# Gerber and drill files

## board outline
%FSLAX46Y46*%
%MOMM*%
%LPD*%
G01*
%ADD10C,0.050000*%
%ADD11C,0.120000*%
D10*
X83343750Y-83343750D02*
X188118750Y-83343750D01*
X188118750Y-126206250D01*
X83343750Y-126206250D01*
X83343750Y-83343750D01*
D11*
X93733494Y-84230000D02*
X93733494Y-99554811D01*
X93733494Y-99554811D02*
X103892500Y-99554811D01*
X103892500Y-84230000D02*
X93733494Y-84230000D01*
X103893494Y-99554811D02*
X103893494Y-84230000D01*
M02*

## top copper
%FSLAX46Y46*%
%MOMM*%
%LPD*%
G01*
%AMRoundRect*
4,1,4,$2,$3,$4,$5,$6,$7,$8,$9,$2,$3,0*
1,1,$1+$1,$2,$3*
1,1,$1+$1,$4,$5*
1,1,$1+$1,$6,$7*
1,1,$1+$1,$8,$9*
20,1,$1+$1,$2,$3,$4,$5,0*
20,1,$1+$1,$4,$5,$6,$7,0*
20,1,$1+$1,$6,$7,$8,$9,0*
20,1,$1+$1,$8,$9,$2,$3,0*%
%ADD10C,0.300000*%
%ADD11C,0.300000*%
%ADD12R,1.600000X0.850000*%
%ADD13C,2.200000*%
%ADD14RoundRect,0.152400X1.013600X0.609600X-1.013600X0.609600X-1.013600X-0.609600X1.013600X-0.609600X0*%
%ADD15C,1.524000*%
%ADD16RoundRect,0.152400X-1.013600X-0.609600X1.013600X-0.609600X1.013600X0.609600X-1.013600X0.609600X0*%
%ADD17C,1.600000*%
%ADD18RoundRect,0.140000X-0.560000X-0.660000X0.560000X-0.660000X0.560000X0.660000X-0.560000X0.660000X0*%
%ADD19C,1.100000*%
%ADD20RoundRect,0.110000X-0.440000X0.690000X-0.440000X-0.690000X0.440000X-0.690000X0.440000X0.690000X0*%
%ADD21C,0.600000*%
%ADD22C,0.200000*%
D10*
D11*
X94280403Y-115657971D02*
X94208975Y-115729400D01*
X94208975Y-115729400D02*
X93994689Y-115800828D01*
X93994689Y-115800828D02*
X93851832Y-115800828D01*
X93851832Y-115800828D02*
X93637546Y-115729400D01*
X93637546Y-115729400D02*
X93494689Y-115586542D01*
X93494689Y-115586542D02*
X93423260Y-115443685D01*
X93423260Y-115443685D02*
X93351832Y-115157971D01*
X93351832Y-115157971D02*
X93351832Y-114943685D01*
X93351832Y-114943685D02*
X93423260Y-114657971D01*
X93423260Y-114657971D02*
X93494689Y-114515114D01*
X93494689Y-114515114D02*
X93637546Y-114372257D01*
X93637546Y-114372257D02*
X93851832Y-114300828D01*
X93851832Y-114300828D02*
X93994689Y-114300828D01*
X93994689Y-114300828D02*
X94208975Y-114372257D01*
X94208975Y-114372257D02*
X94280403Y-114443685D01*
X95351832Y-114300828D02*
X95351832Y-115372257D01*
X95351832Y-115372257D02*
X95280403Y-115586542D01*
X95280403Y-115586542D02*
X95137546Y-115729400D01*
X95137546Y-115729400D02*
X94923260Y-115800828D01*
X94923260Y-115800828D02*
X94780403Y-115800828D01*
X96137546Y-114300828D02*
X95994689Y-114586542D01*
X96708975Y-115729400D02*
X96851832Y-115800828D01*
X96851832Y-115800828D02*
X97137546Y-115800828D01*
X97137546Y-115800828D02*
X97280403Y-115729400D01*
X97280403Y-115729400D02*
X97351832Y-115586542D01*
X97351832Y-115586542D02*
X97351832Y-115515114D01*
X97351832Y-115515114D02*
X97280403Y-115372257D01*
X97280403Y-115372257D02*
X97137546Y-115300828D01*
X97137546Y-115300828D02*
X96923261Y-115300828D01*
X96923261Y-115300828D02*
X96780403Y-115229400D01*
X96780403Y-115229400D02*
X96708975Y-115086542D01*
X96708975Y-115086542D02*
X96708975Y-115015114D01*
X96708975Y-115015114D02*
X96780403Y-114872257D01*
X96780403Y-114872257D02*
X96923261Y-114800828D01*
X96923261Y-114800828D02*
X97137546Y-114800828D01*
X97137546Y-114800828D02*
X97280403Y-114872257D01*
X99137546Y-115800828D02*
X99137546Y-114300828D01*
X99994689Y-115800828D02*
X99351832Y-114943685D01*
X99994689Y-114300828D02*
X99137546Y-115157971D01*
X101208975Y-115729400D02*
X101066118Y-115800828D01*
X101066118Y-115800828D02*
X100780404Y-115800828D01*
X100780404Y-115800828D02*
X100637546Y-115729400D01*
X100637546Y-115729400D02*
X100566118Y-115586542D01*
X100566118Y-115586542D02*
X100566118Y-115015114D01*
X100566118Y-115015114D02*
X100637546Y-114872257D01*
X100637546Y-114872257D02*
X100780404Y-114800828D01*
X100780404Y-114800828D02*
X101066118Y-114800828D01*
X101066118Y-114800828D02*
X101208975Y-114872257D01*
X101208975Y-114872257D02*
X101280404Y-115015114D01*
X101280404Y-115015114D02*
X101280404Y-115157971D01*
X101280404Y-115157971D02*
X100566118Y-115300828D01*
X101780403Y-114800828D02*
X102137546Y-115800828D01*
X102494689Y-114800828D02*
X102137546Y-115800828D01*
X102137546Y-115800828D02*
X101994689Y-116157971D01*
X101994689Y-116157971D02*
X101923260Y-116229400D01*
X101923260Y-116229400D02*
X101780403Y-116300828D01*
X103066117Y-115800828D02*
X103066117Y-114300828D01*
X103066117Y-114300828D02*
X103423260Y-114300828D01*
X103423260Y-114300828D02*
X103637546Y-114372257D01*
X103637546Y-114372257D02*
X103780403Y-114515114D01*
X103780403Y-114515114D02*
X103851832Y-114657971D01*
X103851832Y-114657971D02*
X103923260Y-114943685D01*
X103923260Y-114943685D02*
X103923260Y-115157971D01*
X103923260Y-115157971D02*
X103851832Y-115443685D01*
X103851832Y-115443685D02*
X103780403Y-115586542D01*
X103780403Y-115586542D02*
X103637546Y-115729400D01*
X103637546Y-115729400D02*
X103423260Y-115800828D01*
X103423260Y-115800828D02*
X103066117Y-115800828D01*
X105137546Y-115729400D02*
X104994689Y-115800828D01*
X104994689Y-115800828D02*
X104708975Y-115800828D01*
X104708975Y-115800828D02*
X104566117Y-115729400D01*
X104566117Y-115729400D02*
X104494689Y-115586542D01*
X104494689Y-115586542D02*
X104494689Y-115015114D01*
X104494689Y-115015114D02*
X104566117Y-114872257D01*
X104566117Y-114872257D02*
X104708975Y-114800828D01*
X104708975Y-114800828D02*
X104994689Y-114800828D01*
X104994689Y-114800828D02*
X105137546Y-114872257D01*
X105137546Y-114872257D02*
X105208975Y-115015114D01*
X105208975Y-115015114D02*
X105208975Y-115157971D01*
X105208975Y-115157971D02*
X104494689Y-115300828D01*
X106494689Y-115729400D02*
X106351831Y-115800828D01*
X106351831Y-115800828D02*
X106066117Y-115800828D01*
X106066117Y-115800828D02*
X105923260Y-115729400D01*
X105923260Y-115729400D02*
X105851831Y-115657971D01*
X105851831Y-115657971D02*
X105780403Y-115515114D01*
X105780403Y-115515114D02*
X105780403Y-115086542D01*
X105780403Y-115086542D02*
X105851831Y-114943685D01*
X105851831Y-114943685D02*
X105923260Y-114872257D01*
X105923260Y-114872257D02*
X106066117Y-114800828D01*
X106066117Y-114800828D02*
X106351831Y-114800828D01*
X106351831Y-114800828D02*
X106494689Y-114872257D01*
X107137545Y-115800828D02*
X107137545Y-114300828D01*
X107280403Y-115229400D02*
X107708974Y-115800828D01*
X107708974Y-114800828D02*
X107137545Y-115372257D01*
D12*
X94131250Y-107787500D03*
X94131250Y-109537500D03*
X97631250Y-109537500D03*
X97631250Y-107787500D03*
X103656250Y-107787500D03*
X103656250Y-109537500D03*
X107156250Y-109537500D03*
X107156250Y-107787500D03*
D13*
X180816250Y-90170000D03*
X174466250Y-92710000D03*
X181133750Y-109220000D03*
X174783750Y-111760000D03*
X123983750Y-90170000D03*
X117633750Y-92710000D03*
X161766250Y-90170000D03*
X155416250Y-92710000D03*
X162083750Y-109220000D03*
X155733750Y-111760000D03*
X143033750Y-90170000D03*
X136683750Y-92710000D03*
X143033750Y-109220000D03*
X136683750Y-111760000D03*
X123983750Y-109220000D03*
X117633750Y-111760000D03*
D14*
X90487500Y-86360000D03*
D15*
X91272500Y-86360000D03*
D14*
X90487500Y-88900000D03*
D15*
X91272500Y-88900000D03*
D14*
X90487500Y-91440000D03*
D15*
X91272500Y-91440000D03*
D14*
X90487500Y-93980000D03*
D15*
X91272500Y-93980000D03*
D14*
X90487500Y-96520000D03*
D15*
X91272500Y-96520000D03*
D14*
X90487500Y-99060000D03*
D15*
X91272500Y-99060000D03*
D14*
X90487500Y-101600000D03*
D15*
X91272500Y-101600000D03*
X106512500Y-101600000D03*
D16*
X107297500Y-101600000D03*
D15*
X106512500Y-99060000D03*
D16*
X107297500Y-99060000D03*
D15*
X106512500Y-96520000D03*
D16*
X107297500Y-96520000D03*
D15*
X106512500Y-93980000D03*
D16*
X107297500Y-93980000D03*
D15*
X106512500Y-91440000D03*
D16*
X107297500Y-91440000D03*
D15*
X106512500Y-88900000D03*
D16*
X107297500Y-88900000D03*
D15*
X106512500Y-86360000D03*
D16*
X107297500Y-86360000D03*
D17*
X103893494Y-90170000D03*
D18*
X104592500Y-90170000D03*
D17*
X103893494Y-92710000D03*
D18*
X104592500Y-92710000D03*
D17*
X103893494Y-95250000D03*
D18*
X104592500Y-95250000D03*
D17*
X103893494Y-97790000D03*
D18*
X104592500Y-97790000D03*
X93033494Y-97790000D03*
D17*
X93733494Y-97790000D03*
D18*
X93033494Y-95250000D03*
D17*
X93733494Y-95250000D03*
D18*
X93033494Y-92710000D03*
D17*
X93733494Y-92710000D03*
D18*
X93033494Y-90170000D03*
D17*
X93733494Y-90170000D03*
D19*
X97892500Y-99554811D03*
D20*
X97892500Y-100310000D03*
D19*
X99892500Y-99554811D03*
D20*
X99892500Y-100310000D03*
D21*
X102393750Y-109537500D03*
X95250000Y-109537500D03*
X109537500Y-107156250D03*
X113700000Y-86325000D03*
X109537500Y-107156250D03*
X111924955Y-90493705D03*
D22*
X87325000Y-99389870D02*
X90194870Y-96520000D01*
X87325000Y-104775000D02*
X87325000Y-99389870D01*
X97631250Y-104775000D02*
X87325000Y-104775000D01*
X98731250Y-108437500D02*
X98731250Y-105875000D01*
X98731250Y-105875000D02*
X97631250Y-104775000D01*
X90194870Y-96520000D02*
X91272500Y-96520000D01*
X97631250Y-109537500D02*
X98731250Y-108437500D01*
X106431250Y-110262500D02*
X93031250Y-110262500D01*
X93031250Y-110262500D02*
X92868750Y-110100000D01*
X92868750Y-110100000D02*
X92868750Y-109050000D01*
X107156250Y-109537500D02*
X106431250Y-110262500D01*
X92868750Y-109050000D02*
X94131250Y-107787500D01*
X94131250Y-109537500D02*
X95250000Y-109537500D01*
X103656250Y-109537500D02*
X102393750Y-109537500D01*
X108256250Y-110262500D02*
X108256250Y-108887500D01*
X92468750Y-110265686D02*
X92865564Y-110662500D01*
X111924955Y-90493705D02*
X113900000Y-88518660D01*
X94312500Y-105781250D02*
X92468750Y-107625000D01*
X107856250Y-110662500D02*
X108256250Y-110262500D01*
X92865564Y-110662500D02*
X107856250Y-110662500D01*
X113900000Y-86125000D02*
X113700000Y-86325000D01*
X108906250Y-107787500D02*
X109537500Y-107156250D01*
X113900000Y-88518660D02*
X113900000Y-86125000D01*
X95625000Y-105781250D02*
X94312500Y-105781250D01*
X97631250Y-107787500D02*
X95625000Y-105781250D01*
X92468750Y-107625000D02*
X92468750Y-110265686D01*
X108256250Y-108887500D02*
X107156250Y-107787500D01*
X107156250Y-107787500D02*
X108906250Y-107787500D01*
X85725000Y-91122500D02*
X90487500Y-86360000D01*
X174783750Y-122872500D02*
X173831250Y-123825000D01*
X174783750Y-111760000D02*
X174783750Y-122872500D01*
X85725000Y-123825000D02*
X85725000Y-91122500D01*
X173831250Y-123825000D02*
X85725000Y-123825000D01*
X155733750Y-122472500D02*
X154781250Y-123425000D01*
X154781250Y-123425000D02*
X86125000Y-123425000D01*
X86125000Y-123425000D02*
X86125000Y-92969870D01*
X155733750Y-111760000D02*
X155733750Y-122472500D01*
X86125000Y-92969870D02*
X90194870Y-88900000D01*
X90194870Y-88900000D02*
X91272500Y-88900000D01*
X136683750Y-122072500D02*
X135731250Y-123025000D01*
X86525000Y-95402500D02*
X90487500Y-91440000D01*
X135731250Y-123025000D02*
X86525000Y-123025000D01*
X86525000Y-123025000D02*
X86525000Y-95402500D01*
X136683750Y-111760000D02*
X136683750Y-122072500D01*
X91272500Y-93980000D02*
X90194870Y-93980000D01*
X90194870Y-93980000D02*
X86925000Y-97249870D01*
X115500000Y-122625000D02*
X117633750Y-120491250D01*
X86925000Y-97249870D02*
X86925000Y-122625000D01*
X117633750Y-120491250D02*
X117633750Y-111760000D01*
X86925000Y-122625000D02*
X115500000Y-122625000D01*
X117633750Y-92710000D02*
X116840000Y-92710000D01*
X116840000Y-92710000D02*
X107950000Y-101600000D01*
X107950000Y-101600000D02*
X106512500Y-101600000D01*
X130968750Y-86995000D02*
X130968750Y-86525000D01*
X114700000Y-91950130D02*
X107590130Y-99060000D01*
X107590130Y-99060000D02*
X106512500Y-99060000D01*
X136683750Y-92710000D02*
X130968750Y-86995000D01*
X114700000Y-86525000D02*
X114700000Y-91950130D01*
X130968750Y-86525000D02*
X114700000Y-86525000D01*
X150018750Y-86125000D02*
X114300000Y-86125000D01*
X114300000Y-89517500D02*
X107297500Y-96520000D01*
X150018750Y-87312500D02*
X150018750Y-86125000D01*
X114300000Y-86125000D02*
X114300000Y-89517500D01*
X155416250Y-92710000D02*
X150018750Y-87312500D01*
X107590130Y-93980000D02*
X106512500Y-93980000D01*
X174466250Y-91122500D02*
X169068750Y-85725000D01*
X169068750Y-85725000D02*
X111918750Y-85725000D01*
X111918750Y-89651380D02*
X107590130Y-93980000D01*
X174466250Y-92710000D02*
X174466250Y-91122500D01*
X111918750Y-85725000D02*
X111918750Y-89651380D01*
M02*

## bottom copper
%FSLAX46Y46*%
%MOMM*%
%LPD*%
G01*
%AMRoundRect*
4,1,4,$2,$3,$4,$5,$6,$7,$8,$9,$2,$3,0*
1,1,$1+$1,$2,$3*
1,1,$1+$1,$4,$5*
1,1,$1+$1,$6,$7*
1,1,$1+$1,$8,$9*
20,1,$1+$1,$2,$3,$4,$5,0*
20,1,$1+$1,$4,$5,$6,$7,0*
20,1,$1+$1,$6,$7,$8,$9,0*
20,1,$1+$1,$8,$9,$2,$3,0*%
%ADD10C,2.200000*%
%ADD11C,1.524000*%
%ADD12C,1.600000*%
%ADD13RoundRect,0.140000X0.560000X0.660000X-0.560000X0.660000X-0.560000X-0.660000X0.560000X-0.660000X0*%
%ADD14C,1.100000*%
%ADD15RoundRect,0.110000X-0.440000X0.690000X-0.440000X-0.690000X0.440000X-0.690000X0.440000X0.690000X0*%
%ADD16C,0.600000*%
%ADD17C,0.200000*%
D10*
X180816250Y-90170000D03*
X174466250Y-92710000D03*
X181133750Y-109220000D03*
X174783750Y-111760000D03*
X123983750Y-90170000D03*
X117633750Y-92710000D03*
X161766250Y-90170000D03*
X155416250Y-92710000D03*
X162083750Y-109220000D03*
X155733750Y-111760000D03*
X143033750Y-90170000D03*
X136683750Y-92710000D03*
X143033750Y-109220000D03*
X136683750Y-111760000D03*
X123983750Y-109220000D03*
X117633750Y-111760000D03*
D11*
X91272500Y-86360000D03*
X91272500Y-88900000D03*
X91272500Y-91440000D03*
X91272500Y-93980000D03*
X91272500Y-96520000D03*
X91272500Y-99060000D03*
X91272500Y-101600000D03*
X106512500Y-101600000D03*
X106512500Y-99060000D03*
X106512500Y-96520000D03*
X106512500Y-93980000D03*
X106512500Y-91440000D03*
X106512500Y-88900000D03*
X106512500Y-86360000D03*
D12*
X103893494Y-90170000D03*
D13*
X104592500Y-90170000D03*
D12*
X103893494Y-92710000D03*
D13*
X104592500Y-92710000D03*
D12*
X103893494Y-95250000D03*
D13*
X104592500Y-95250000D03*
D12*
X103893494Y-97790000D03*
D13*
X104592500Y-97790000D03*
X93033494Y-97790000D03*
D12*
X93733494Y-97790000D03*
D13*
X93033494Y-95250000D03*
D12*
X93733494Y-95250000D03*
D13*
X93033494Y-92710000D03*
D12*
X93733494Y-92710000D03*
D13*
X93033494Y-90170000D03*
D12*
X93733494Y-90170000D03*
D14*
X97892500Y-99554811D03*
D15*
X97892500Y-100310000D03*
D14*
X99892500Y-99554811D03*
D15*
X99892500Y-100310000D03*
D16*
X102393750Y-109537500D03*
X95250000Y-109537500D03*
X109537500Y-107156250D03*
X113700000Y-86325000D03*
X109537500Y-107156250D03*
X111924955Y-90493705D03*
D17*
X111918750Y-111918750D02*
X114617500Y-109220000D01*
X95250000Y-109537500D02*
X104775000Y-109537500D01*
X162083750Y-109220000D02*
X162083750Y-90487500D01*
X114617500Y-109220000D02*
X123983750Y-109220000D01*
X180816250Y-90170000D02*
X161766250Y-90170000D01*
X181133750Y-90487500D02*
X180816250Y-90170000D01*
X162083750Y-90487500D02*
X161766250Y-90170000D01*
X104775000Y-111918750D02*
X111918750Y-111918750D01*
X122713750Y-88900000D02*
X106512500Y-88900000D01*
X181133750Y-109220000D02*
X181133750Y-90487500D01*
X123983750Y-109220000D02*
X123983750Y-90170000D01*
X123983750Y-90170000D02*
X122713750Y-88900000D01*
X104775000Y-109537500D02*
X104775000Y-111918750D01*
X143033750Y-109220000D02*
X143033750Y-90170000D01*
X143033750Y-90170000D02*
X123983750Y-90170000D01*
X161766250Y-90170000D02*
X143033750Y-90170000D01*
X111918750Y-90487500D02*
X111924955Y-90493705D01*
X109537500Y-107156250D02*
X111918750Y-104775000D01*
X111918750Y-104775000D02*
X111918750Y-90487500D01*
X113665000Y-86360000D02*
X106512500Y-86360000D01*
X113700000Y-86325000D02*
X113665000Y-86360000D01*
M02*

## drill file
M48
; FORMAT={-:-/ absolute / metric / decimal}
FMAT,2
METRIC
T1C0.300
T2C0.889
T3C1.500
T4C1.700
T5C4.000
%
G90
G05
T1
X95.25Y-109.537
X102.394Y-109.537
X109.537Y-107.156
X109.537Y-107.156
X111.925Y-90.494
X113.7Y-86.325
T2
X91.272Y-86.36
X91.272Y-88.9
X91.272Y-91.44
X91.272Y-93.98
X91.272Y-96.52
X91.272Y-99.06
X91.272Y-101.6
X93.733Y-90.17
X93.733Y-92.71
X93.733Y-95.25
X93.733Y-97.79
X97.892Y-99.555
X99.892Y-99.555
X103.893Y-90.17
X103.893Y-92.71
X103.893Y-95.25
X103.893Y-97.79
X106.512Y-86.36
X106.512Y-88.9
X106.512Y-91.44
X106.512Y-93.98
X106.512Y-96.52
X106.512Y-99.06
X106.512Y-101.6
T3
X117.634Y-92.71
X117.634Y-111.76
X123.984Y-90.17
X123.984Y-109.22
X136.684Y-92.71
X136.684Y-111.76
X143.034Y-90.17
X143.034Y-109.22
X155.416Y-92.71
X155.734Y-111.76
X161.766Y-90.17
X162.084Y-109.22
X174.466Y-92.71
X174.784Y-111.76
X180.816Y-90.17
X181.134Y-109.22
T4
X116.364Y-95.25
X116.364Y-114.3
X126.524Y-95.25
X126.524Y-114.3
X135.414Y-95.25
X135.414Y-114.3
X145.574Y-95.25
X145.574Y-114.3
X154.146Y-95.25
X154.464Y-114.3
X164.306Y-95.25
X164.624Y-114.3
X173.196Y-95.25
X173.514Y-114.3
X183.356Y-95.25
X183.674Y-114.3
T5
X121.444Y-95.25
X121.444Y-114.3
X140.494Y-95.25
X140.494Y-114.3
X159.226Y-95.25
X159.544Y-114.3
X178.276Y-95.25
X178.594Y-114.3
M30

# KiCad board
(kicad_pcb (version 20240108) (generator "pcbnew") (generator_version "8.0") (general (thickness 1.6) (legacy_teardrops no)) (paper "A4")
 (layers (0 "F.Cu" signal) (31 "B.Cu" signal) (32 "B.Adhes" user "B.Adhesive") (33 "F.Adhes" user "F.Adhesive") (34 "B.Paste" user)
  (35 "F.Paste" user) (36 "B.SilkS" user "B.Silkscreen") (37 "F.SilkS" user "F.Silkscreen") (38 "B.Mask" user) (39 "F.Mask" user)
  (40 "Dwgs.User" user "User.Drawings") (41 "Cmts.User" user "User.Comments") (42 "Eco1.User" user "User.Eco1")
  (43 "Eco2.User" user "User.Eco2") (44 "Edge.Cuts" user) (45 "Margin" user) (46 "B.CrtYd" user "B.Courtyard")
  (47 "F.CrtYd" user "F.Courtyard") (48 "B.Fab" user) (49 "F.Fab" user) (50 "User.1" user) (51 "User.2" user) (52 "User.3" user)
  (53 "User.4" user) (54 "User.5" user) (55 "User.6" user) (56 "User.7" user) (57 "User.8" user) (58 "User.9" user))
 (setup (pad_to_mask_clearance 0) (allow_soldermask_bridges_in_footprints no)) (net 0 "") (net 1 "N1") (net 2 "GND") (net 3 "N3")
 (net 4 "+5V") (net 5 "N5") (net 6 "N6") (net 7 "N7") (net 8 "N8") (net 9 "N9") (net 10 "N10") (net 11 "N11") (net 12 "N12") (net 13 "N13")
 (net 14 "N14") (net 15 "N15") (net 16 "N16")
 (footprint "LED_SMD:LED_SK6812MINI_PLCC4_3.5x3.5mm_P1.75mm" (layer "F.Cu") (at 95.88125 108.6625)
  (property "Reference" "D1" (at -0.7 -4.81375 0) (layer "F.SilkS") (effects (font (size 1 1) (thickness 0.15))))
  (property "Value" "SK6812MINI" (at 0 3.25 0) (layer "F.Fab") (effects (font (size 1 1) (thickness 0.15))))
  (pad "1" smd rect (at -1.75 -0.875) (size 1.6 0.85) (layers "F.Cu" "F.Paste" "F.Mask") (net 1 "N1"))
  (pad "2" smd rect (at -1.75 0.875) (size 1.6 0.85) (layers "F.Cu" "F.Paste" "F.Mask") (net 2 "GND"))
  (pad "3" smd rect (at 1.75 0.875) (size 1.6 0.85) (layers "F.Cu" "F.Paste" "F.Mask") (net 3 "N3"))
  (pad "4" smd rect (at 1.75 -0.875) (size 1.6 0.85) (layers "F.Cu" "F.Paste" "F.Mask") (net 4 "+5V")))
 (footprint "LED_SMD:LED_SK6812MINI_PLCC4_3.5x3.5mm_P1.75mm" (layer "F.Cu") (at 105.40625 108.6625)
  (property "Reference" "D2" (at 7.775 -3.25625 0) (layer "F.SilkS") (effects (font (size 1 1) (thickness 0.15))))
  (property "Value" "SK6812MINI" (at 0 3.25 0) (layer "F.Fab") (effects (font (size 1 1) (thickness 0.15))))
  (pad "1" smd rect (at -1.75 -0.875) (size 1.6 0.85) (layers "F.Cu" "F.Paste" "F.Mask") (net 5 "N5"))
  (pad "2" smd rect (at -1.75 0.875) (size 1.6 0.85) (layers "F.Cu" "F.Paste" "F.Mask") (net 2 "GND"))
  (pad "3" smd rect (at 1.75 0.875) (size 1.6 0.85) (layers "F.Cu" "F.Paste" "F.Mask") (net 1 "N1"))
  (pad "4" smd rect (at 1.75 -0.875) (size 1.6 0.85) (layers "F.Cu" "F.Paste" "F.Mask") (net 4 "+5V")))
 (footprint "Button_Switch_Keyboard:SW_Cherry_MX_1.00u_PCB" (layer "F.Cu") (at 180.81625 90.17)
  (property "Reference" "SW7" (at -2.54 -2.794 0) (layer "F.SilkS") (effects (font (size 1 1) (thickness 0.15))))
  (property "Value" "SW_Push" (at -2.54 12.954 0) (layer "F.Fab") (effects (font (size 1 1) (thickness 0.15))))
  (pad "" np_thru_hole circle (at -7.62 5.08) (size 1.7 1.7) (drill 1.7) (layers "*.Cu" "*.Mask"))
  (pad "" np_thru_hole circle (at -2.54 5.08) (size 4 4) (drill 4) (layers "*.Cu" "*.Mask"))
  (pad "" np_thru_hole circle (at 2.54 5.08) (size 1.7 1.7) (drill 1.7) (layers "*.Cu" "*.Mask"))
  (pad "1" thru_hole circle (at 0 0) (size 2.2 2.2) (drill 1.5) (layers "*.Cu" "*.Mask") (remove_unused_layers no) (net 2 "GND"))
  (pad "2" thru_hole circle (at -6.35 2.54) (size 2.2 2.2) (drill 1.5) (layers "*.Cu" "*.Mask") (remove_unused_layers no) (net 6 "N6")))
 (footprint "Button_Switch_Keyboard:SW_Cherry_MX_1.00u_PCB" (layer "F.Cu") (at 181.13375 109.22)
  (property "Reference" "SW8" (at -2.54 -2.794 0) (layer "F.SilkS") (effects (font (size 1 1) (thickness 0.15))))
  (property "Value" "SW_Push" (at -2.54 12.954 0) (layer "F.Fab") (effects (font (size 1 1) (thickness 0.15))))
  (pad "" np_thru_hole circle (at -7.62 5.08) (size 1.7 1.7) (drill 1.7) (layers "*.Cu" "*.Mask"))
  (pad "" np_thru_hole circle (at -2.54 5.08) (size 4 4) (drill 4) (layers "*.Cu" "*.Mask"))
  (pad "" np_thru_hole circle (at 2.54 5.08) (size 1.7 1.7) (drill 1.7) (layers "*.Cu" "*.Mask"))
  (pad "1" thru_hole circle (at 0 0) (size 2.2 2.2) (drill 1.5) (layers "*.Cu" "*.Mask") (remove_unused_layers no) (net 2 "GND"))
  (pad "2" thru_hole circle (at -6.35 2.54) (size 2.2 2.2) (drill 1.5) (layers "*.Cu" "*.Mask") (remove_unused_layers no) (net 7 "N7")))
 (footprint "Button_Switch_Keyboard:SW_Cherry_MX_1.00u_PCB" (layer "F.Cu") (at 123.98375 90.17)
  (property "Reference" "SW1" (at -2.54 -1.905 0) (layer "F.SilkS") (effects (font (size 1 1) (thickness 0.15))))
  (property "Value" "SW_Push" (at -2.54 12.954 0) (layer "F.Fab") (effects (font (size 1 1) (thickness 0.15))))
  (pad "" np_thru_hole circle (at -7.62 5.08) (size 1.7 1.7) (drill 1.7) (layers "*.Cu" "*.Mask"))
  (pad "" np_thru_hole circle (at -2.54 5.08) (size 4 4) (drill 4) (layers "*.Cu" "*.Mask"))
  (pad "" np_thru_hole circle (at 2.54 5.08) (size 1.7 1.7) (drill 1.7) (layers "*.Cu" "*.Mask"))
  (pad "1" thru_hole circle (at 0 0) (size 2.2 2.2) (drill 1.5) (layers "*.Cu" "*.Mask") (remove_unused_layers no) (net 2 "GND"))
  (pad "2" thru_hole circle (at -6.35 2.54) (size 2.2 2.2) (drill 1.5) (layers "*.Cu" "*.Mask") (remove_unused_layers no) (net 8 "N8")))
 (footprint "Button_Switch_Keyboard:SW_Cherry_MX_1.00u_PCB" (layer "F.Cu") (at 161.76625 90.17)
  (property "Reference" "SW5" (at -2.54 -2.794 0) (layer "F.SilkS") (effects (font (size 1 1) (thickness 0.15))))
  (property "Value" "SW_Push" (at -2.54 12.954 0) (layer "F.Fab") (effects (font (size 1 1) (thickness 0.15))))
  (pad "" np_thru_hole circle (at -7.62 5.08) (size 1.7 1.7) (drill 1.7) (layers "*.Cu" "*.Mask"))
  (pad "" np_thru_hole circle (at -2.54 5.08) (size 4 4) (drill 4) (layers "*.Cu" "*.Mask"))
  (pad "" np_thru_hole circle (at 2.54 5.08) (size 1.7 1.7) (drill 1.7) (layers "*.Cu" "*.Mask"))
  (pad "1" thru_hole circle (at 0 0) (size 2.2 2.2) (drill 1.5) (layers "*.Cu" "*.Mask") (remove_unused_layers no) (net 2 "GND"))
  (pad "2" thru_hole circle (at -6.35 2.54) (size 2.2 2.2) (drill 1.5) (layers "*.Cu" "*.Mask") (remove_unused_layers no) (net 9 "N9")))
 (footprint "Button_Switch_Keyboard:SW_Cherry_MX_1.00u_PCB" (layer "F.Cu") (at 162.08375 109.22)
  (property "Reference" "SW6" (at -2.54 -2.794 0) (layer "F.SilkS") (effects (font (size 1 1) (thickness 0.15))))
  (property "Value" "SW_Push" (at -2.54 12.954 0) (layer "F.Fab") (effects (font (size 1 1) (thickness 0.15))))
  (pad "" np_thru_hole circle (at -7.62 5.08) (size 1.7 1.7) (drill 1.7) (layers "*.Cu" "*.Mask"))
  (pad "" np_thru_hole circle (at -2.54 5.08) (size 4 4) (drill 4) (layers "*.Cu" "*.Mask"))
  (pad "" np_thru_hole circle (at 2.54 5.08) (size 1.7 1.7) (drill 1.7) (layers "*.Cu" "*.Mask"))
  (pad "1" thru_hole circle (at 0 0) (size 2.2 2.2) (drill 1.5) (layers "*.Cu" "*.Mask") (remove_unused_layers no) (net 2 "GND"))
  (pad "2" thru_hole circle (at -6.35 2.54) (size 2.2 2.2) (drill 1.5) (layers "*.Cu" "*.Mask") (remove_unused_layers no) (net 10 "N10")))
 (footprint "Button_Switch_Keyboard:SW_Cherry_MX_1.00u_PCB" (layer "F.Cu") (at 143.03375 90.17)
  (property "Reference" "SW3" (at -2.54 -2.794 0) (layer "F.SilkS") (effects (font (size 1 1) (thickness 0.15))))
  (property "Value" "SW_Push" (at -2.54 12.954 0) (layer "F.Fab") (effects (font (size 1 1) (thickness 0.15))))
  (pad "" np_thru_hole circle (at -7.62 5.08) (size 1.7 1.7) (drill 1.7) (layers "*.Cu" "*.Mask"))
  (pad "" np_thru_hole circle (at -2.54 5.08) (size 4 4) (drill 4) (layers "*.Cu" "*.Mask"))
  (pad "" np_thru_hole circle (at 2.54 5.08) (size 1.7 1.7) (drill 1.7) (layers "*.Cu" "*.Mask"))
  (pad "1" thru_hole circle (at 0 0) (size 2.2 2.2) (drill 1.5) (layers "*.Cu" "*.Mask") (remove_unused_layers no) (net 2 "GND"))
  (pad "2" thru_hole circle (at -6.35 2.54) (size 2.2 2.2) (drill 1.5) (layers "*.Cu" "*.Mask") (remove_unused_layers no) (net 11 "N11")))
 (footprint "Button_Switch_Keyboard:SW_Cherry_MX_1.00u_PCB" (layer "F.Cu") (at 143.03375 109.22)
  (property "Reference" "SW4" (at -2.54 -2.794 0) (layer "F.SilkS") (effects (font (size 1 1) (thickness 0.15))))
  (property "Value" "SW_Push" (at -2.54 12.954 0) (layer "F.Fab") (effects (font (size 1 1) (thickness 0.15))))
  (pad "" np_thru_hole circle (at -7.62 5.08) (size 1.7 1.7) (drill 1.7) (layers "*.Cu" "*.Mask"))
  (pad "" np_thru_hole circle (at -2.54 5.08) (size 4 4) (drill 4) (layers "*.Cu" "*.Mask"))
  (pad "" np_thru_hole circle (at 2.54 5.08) (size 1.7 1.7) (drill 1.7) (layers "*.Cu" "*.Mask"))
  (pad "1" thru_hole circle (at 0 0) (size 2.2 2.2) (drill 1.5) (layers "*.Cu" "*.Mask") (remove_unused_layers no) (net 2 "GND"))
  (pad "2" thru_hole circle (at -6.35 2.54) (size 2.2 2.2) (drill 1.5) (layers "*.Cu" "*.Mask") (remove_unused_layers no) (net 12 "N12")))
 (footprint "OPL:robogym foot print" (layer "F.Cu") (at 100.0125 119.0625)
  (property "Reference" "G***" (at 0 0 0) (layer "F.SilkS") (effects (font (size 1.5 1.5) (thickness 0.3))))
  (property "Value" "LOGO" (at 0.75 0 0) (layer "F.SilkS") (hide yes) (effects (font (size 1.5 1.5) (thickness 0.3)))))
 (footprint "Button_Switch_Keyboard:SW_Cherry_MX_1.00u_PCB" (layer "F.Cu") (at 123.98375 109.22)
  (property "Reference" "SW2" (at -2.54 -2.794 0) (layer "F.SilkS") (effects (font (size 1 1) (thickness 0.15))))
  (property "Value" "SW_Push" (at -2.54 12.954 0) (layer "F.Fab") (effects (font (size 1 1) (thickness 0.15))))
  (pad "" np_thru_hole circle (at -7.62 5.08) (size 1.7 1.7) (drill 1.7) (layers "*.Cu" "*.Mask"))
  (pad "" np_thru_hole circle (at -2.54 5.08) (size 4 4) (drill 4) (layers "*.Cu" "*.Mask"))
  (pad "" np_thru_hole circle (at 2.54 5.08) (size 1.7 1.7) (drill 1.7) (layers "*.Cu" "*.Mask"))
  (pad "1" thru_hole circle (at 0 0) (size 2.2 2.2) (drill 1.5) (layers "*.Cu" "*.Mask") (remove_unused_layers no) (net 2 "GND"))
  (pad "2" thru_hole circle (at -6.35 2.54) (size 2.2 2.2) (drill 1.5) (layers "*.Cu" "*.Mask") (remove_unused_layers no) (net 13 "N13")))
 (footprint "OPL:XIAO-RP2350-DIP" (layer "F.Cu") (at 98.893494 93.9165)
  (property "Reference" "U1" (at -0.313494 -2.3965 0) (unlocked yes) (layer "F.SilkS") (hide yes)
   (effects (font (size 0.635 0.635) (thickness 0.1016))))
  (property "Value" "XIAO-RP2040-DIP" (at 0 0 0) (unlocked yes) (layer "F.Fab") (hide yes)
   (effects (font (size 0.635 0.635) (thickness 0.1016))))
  (fp_line (start -5.16 -9.6865) (end -5.16 5.638311) (stroke (width 0.12) (type default)) (layer "Edge.Cuts"))
  (fp_line (start -5.16 5.638311) (end 4.999006 5.638311) (stroke (width 0.12) (type default)) (layer "Edge.Cuts"))
  (fp_line (start 4.999006 -9.6865) (end -5.16 -9.6865) (stroke (width 0.12) (type default)) (layer "Edge.Cuts"))
  (fp_line (start 5 5.638311) (end 5 -9.6865) (stroke (width 0.12) (type default)) (layer "Edge.Cuts"))
  (pad "1" smd roundrect (at -8.405994 -7.5565 180) (size 2.332 1.524) (layers "F.Cu" "F.Mask") (roundrect_rratio 0.1) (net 7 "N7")
   (thermal_bridge_angle 45))
  (pad "1" thru_hole circle (at -7.620994 -7.5565 180) (size 1.524 1.524) (drill 0.889) (layers "*.Cu" "*.Mask") (remove_unused_layers no)
   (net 7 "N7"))
  (pad "2" smd roundrect (at -8.405994 -5.0165 180) (size 2.332 1.524) (layers "F.Cu" "F.Mask") (roundrect_rratio 0.1) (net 10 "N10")
   (thermal_bridge_angle 45))
  (pad "2" thru_hole circle (at -7.620994 -5.0165 180) (size 1.524 1.524) (drill 0.889) (layers "*.Cu" "*.Mask") (remove_unused_layers no)
   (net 10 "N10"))
  (pad "3" smd roundrect (at -8.405994 -2.4765 180) (size 2.332 1.524) (layers "F.Cu" "F.Mask") (roundrect_rratio 0.1) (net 12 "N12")
   (thermal_bridge_angle 45))
  (pad "3" thru_hole circle (at -7.620994 -2.4765 180) (size 1.524 1.524) (drill 0.889) (layers "*.Cu" "*.Mask") (remove_unused_layers no)
   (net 12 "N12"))
  (pad "4" smd roundrect (at -8.405994 0.0635 180) (size 2.332 1.524) (layers "F.Cu" "F.Mask") (roundrect_rratio 0.1) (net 13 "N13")
   (thermal_bridge_angle 45))
  (pad "4" thru_hole circle (at -7.620994 0.0635 180) (size 1.524 1.524) (drill 0.889) (layers "*.Cu" "*.Mask") (remove_unused_layers no)
   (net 13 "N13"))
  (pad "5" smd roundrect (at -8.405994 2.6035 180) (size 2.332 1.524) (layers "F.Cu" "F.Mask") (roundrect_rratio 0.1) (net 3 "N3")
   (thermal_bridge_angle 45))
  (pad "5" thru_hole circle (at -7.620994 2.6035 180) (size 1.524 1.524) (drill 0.889) (layers "*.Cu" "*.Mask") (remove_unused_layers no)
   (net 3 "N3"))
  (pad "6" smd roundrect (at -8.405994 5.1435 180) (size 2.332 1.524) (layers "F.Cu" "F.Mask") (roundrect_rratio 0.1) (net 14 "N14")
   (thermal_bridge_angle 45))
  (pad "6" thru_hole circle (at -7.620994 5.1435 180) (size 1.524 1.524) (drill 0.889) (layers "*.Cu" "*.Mask") (remove_unused_layers no)
   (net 14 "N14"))
  (pad "7" smd roundrect (at -8.405994 7.6835 180) (size 2.332 1.524) (layers "F.Cu" "F.Mask") (roundrect_rratio 0.1) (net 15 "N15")
   (thermal_bridge_angle 45))
  (pad "7" thru_hole circle (at -7.620994 7.6835 180) (size 1.524 1.524) (drill 0.889) (layers "*.Cu" "*.Mask") (remove_unused_layers no)
   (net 15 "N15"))
  (pad "8" thru_hole circle (at 7.619006 7.6835) (size 1.524 1.524) (drill 0.889) (layers "*.Cu" "*.Mask") (remove_unused_layers no)
   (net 8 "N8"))
  (pad "8" smd roundrect (at 8.404006 7.6835) (size 2.332 1.524) (layers "F.Cu" "F.Mask") (roundrect_rratio 0.1) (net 8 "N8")
   (thermal_bridge_angle 45))
  (pad "9" thru_hole circle (at 7.619006 5.1435) (size 1.524 1.524) (drill 0.889) (layers "*.Cu" "*.Mask") (remove_unused_layers no)
   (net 11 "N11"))
  (pad "9" smd roundrect (at 8.404006 5.1435) (size 2.332 1.524) (layers "F.Cu" "F.Mask") (roundrect_rratio 0.1) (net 11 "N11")
   (thermal_bridge_angle 45))
  (pad "10" thru_hole circle (at 7.619006 2.6035) (size 1.524 1.524) (drill 0.889) (layers "*.Cu" "*.Mask") (remove_unused_layers no)
   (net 9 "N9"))
  (pad "10" smd roundrect (at 8.404006 2.6035) (size 2.332 1.524) (layers "F.Cu" "F.Mask") (roundrect_rratio 0.1) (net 9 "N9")
   (thermal_bridge_angle 45))
  (pad "11" thru_hole circle (at 7.619006 0.0635) (size 1.524 1.524) (drill 0.889) (layers "*.Cu" "*.Mask") (remove_unused_layers no)
   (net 6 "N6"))
  (pad "11" smd roundrect (at 8.404006 0.0635) (size 2.332 1.524) (layers "F.Cu" "F.Mask") (roundrect_rratio 0.1) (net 6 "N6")
   (thermal_bridge_angle 45))
  (pad "12" thru_hole circle (at 7.619006 -2.4765) (size 1.524 1.524) (drill 0.889) (layers "*.Cu" "*.Mask") (remove_unused_layers no)
   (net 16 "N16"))
  (pad "12" smd roundrect (at 8.404006 -2.4765) (size 2.332 1.524) (layers "F.Cu" "F.Mask") (roundrect_rratio 0.1) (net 16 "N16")
   (thermal_bridge_angle 45))
  (pad "13" thru_hole circle (at 7.619006 -5.0165) (size 1.524 1.524) (drill 0.889) (layers "*.Cu" "*.Mask") (remove_unused_layers no)
   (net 2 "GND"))
  (pad "13" smd roundrect (at 8.404006 -5.0165) (size 2.332 1.524) (layers "F.Cu" "F.Mask") (roundrect_rratio 0.1) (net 2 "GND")
   (thermal_bridge_angle 45))
  (pad "14" thru_hole circle (at 7.619006 -7.5565) (size 1.524 1.524) (drill 0.889) (layers "*.Cu" "*.Mask") (remove_unused_layers no)
   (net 4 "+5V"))
  (pad "14" smd roundrect (at 8.404006 -7.5565) (size 2.332 1.524) (layers "F.Cu" "F.Mask") (roundrect_rratio 0.1) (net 4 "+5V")
   (thermal_bridge_angle 45))
  (pad "15" thru_hole circle (at 5 -3.7465 180) (size 1.6 1.6) (drill 0.889) (layers "*.Cu" "*.Mask") (remove_unused_layers no))
  (pad "15" smd roundrect (at 5.699006 -3.7465) (size 1.4 1.6) (layers "F.Cu" "F.Mask") (roundrect_rratio 0.1) (thermal_bridge_angle 45))
  (pad "15" smd roundrect (at 5.699006 -3.7465 180) (size 1.4 1.6) (layers "B.Cu" "B.Paste" "B.Mask") (roundrect_rratio 0.1)
   (thermal_bridge_angle 45))
  (pad "16" thru_hole circle (at 5 -1.2065 180) (size 1.6 1.6) (drill 0.889) (layers "*.Cu" "*.Mask") (remove_unused_layers no))
  (pad "16" smd roundrect (at 5.699006 -1.2065) (size 1.4 1.6) (layers "F.Cu" "F.Mask") (roundrect_rratio 0.1) (thermal_bridge_angle 45))
  (pad "16" smd roundrect (at 5.699006 -1.2065 180) (size 1.4 1.6) (layers "B.Cu" "B.Paste" "B.Mask") (roundrect_rratio 0.1)
   (thermal_bridge_angle 45))
  (pad "17" thru_hole circle (at 5 1.3335 180) (size 1.6 1.6) (drill 0.889) (layers "*.Cu" "*.Mask") (remove_unused_layers no))
  (pad "17" smd roundrect (at 5.699006 1.3335) (size 1.4 1.6) (layers "F.Cu" "F.Mask") (roundrect_rratio 0.1) (thermal_bridge_angle 45))
  (pad "17" smd roundrect (at 5.699006 1.3335 180) (size 1.4 1.6) (layers "B.Cu" "B.Paste" "B.Mask") (roundrect_rratio 0.1)
   (thermal_bridge_angle 45))
  (pad "18" thru_hole circle (at 5 3.8735 180) (size 1.6 1.6) (drill 0.889) (layers "*.Cu" "*.Mask") (remove_unused_layers no))
  (pad "18" smd roundrect (at 5.699006 3.8735) (size 1.4 1.6) (layers "F.Cu" "F.Mask") (roundrect_rratio 0.1) (thermal_bridge_angle 45))
  (pad "18" smd roundrect (at 5.699006 3.8735 180) (size 1.4 1.6) (layers "B.Cu" "B.Paste" "B.Mask") (roundrect_rratio 0.1)
   (thermal_bridge_angle 45))
  (pad "19" smd roundrect (at -5.86 3.8735) (size 1.4 1.6) (layers "F.Cu" "F.Mask") (roundrect_rratio 0.1) (thermal_bridge_angle 45))
  (pad "19" smd roundrect (at -5.86 3.8735 180) (size 1.4 1.6) (layers "B.Cu" "B.Paste" "B.Mask") (roundrect_rratio 0.1)
   (thermal_bridge_angle 45))
  (pad "19" thru_hole circle (at -5.16 3.8735 180) (size 1.6 1.6) (drill 0.889) (layers "*.Cu" "*.Mask") (remove_unused_layers no))
  (pad "20" smd roundrect (at -5.86 1.3335) (size 1.4 1.6) (layers "F.Cu" "F.Mask") (roundrect_rratio 0.1) (thermal_bridge_angle 45))
  (pad "20" smd roundrect (at -5.86 1.3335 180) (size 1.4 1.6) (layers "B.Cu" "B.Paste" "B.Mask") (roundrect_rratio 0.1)
   (thermal_bridge_angle 45))
  (pad "20" thru_hole circle (at -5.16 1.3335 180) (size 1.6 1.6) (drill 0.889) (layers "*.Cu" "*.Mask") (remove_unused_layers no))
  (pad "21" smd roundrect (at -5.86 -1.2065) (size 1.4 1.6) (layers "F.Cu" "F.Mask") (roundrect_rratio 0.1) (thermal_bridge_angle 45))
  (pad "21" smd roundrect (at -5.86 -1.2065 180) (size 1.4 1.6) (layers "B.Cu" "B.Paste" "B.Mask") (roundrect_rratio 0.1)
   (thermal_bridge_angle 45))
  (pad "21" thru_hole circle (at -5.16 -1.2065 180) (size 1.6 1.6) (drill 0.889) (layers "*.Cu" "*.Mask") (remove_unused_layers no))
  (pad "22" smd roundrect (at -5.86 -3.7465) (size 1.4 1.6) (layers "F.Cu" "F.Mask") (roundrect_rratio 0.1) (thermal_bridge_angle 45))
  (pad "22" smd roundrect (at -5.86 -3.7465 180) (size 1.4 1.6) (layers "B.Cu" "B.Paste" "B.Mask") (roundrect_rratio 0.1)
   (thermal_bridge_angle 45))
  (pad "22" thru_hole circle (at -5.16 -3.7465 180) (size 1.6 1.6) (drill 0.889) (layers "*.Cu" "*.Mask") (remove_unused_layers no))
  (pad "23" thru_hole circle (at -1.000994 5.638311 180) (size 1.1 1.1) (drill 0.889) (layers "*.Cu" "*.Mask") (remove_unused_layers no))
  (pad "23" smd roundrect (at -1.000994 6.3935 270) (size 1.6 1.1) (layers "F.Cu" "F.Mask") (roundrect_rratio 0.1) (thermal_bridge_angle 45))
  (pad "23" smd roundrect (at -1.000994 6.3935 270) (size 1.6 1.1) (layers "B.Cu" "B.Paste" "B.Mask") (roundrect_rratio 0.1)
   (thermal_bridge_angle 45))
  (pad "24" thru_hole circle (at 0.999006 5.638311 180) (size 1.1 1.1) (drill 0.889) (layers "*.Cu" "*.Mask") (remove_unused_layers no))
  (pad "24" smd roundrect (at 0.999006 6.3935 270) (size 1.6 1.1) (layers "F.Cu" "F.Mask") (roundrect_rratio 0.1) (thermal_bridge_angle 45))
  (pad "24" smd roundrect (at 0.999006 6.3935 270) (size 1.6 1.1) (layers "B.Cu" "B.Paste" "B.Mask") (roundrect_rratio 0.1)
   (thermal_bridge_angle 45)))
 (gr_rect (start 83.34375 83.34375) (end 188.11875 126.20625) (stroke (width 0.05) (type default)) (fill none) (layer "Edge.Cuts"))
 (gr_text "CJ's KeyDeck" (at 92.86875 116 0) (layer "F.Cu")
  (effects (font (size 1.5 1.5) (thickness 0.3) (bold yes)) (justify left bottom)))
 (segment (start 87.325 99.38987) (end 90.19487 96.52) (width 0.2) (layer "F.Cu") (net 3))
 (segment (start 87.325 104.775) (end 87.325 99.38987) (width 0.2) (layer "F.Cu") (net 3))
 (segment (start 97.63125 104.775) (end 87.325 104.775) (width 0.2) (layer "F.Cu") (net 3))
 (segment (start 98.73125 108.4375) (end 98.73125 105.875) (width 0.2) (layer "F.Cu") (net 3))
 (segment (start 98.73125 105.875) (end 97.63125 104.775) (width 0.2) (layer "F.Cu") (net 3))
 (segment (start 90.19487 96.52) (end 91.2725 96.52) (width 0.2) (layer "F.Cu") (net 3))
 (segment (start 97.63125 109.5375) (end 98.73125 108.4375) (width 0.2) (layer "F.Cu") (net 3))
 (segment (start 106.43125 110.2625) (end 93.03125 110.2625) (width 0.2) (layer "F.Cu") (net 1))
 (segment (start 93.03125 110.2625) (end 92.86875 110.1) (width 0.2) (layer "F.Cu") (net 1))
 (segment (start 92.86875 110.1) (end 92.86875 109.05) (width 0.2) (layer "F.Cu") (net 1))
 (segment (start 107.15625 109.5375) (end 106.43125 110.2625) (width 0.2) (layer "F.Cu") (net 1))
 (segment (start 92.86875 109.05) (end 94.13125 107.7875) (width 0.2) (layer "F.Cu") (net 1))
 (segment (start 94.13125 109.5375) (end 95.25 109.5375) (width 0.2) (layer "F.Cu") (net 2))
 (segment (start 103.65625 109.5375) (end 102.39375 109.5375) (width 0.2) (layer "F.Cu") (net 2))
 (via (at 102.39375 109.5375) (size 0.6) (drill 0.3) (layers "F.Cu" "B.Cu") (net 2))
 (via (at 95.25 109.5375) (size 0.6) (drill 0.3) (layers "F.Cu" "B.Cu") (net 2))
 (segment (start 111.91875 111.91875) (end 114.6175 109.22) (width 0.2) (layer "B.Cu") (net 2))
 (segment (start 95.25 109.5375) (end 104.775 109.5375) (width 0.2) (layer "B.Cu") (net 2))
 (segment (start 162.08375 109.22) (end 162.08375 90.4875) (width 0.2) (layer "B.Cu") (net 2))
 (segment (start 114.6175 109.22) (end 123.98375 109.22) (width 0.2) (layer "B.Cu") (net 2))
 (segment (start 180.81625 90.17) (end 161.76625 90.17) (width 0.2) (layer "B.Cu") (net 2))
 (segment (start 181.13375 90.4875) (end 180.81625 90.17) (width 0.2) (layer "B.Cu") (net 2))
 (segment (start 162.08375 90.4875) (end 161.76625 90.17) (width 0.2) (layer "B.Cu") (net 2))
 (segment (start 104.775 111.91875) (end 111.91875 111.91875) (width 0.2) (layer "B.Cu") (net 2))
 (segment (start 122.71375 88.9) (end 106.5125 88.9) (width 0.2) (layer "B.Cu") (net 2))
 (segment (start 181.13375 109.22) (end 181.13375 90.4875) (width 0.2) (layer "B.Cu") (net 2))
 (segment (start 123.98375 109.22) (end 123.98375 90.17) (width 0.2) (layer "B.Cu") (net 2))
 (segment (start 123.98375 90.17) (end 122.71375 88.9) (width 0.2) (layer "B.Cu") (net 2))
 (segment (start 104.775 109.5375) (end 104.775 111.91875) (width 0.2) (layer "B.Cu") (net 2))
 (segment (start 143.03375 109.22) (end 143.03375 90.17) (width 0.2) (layer "B.Cu") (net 2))
 (segment (start 143.03375 90.17) (end 123.98375 90.17) (width 0.2) (layer "B.Cu") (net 2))
 (segment (start 161.76625 90.17) (end 143.03375 90.17) (width 0.2) (layer "B.Cu") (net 2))
 (segment (start 108.25625 110.2625) (end 108.25625 108.8875) (width 0.2) (layer "F.Cu") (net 4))
 (segment (start 92.46875 110.265686) (end 92.865564 110.6625) (width 0.2) (layer "F.Cu") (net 4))
 (segment (start 111.924955 90.493705) (end 113.9 88.51866) (width 0.2) (layer "F.Cu") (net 4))
 (segment (start 94.3125 105.78125) (end 92.46875 107.625) (width 0.2) (layer "F.Cu") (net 4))
 (segment (start 107.85625 110.6625) (end 108.25625 110.2625) (width 0.2) (layer "F.Cu") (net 4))
 (segment (start 92.865564 110.6625) (end 107.85625 110.6625) (width 0.2) (layer "F.Cu") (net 4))
 (segment (start 113.9 86.125) (end 113.7 86.325) (width 0.2) (layer "F.Cu") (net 4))
 (segment (start 108.90625 107.7875) (end 109.5375 107.15625) (width 0.2) (layer "F.Cu") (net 4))
 (segment (start 113.9 88.51866) (end 113.9 86.125) (width 0.2) (layer "F.Cu") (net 4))
 (segment (start 95.625 105.78125) (end 94.3125 105.78125) (width 0.2) (layer "F.Cu") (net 4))
 (segment (start 97.63125 107.7875) (end 95.625 105.78125) (width 0.2) (layer "F.Cu") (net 4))
 (segment (start 92.46875 107.625) (end 92.46875 110.265686) (width 0.2) (layer "F.Cu") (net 4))
 (segment (start 108.25625 108.8875) (end 107.15625 107.7875) (width 0.2) (layer "F.Cu") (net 4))
 (segment (start 107.15625 107.7875) (end 108.90625 107.7875) (width 0.2) (layer "F.Cu") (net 4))
 (via (at 109.5375 107.15625) (size 0.6) (drill 0.3) (layers "F.Cu" "B.Cu") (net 4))
 (via (at 113.7 86.325) (size 0.6) (drill 0.3) (layers "F.Cu" "B.Cu") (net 4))
 (via (at 109.5375 107.15625) (size 0.6) (drill 0.3) (layers "F.Cu" "B.Cu") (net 4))
 (via (at 111.924955 90.493705) (size 0.6) (drill 0.3) (layers "F.Cu" "B.Cu") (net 4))
 (segment (start 111.91875 90.4875) (end 111.924955 90.493705) (width 0.2) (layer "B.Cu") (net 4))
 (segment (start 109.5375 107.15625) (end 111.91875 104.775) (width 0.2) (layer "B.Cu") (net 4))
 (segment (start 111.91875 104.775) (end 111.91875 90.4875) (width 0.2) (layer "B.Cu") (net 4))
 (segment (start 113.665 86.36) (end 106.5125 86.36) (width 0.2) (layer "B.Cu") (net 4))
 (segment (start 113.7 86.325) (end 113.665 86.36) (width 0.2) (layer "B.Cu") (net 4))
 (segment (start 85.725 91.1225) (end 90.4875 86.36) (width 0.2) (layer "F.Cu") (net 7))
 (segment (start 174.78375 122.8725) (end 173.83125 123.825) (width 0.2) (layer "F.Cu") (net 7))
 (segment (start 174.78375 111.76) (end 174.78375 122.8725) (width 0.2) (layer "F.Cu") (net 7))
 (segment (start 85.725 123.825) (end 85.725 91.1225) (width 0.2) (layer "F.Cu") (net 7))
 (segment (start 173.83125 123.825) (end 85.725 123.825) (width 0.2) (layer "F.Cu") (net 7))
 (segment (start 155.73375 122.4725) (end 154.78125 123.425) (width 0.2) (layer "F.Cu") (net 10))
 (segment (start 154.78125 123.425) (end 86.125 123.425) (width 0.2) (layer "F.Cu") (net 10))
 (segment (start 86.125 123.425) (end 86.125 92.96987) (width 0.2) (layer "F.Cu") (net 10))
 (segment (start 155.73375 111.76) (end 155.73375 122.4725) (width 0.2) (layer "F.Cu") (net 10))
 (segment (start 86.125 92.96987) (end 90.19487 88.9) (width 0.2) (layer "F.Cu") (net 10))
 (segment (start 90.19487 88.9) (end 91.2725 88.9) (width 0.2) (layer "F.Cu") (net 10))
 (segment (start 136.68375 122.0725) (end 135.73125 123.025) (width 0.2) (layer "F.Cu") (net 12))
 (segment (start 86.525 95.4025) (end 90.4875 91.44) (width 0.2) (layer "F.Cu") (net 12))
 (segment (start 135.73125 123.025) (end 86.525 123.025) (width 0.2) (layer "F.Cu") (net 12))
 (segment (start 86.525 123.025) (end 86.525 95.4025) (width 0.2) (layer "F.Cu") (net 12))
 (segment (start 136.68375 111.76) (end 136.68375 122.0725) (width 0.2) (layer "F.Cu") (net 12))
 (segment (start 91.2725 93.98) (end 90.19487 93.98) (width 0.2) (layer "F.Cu") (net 13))
 (segment (start 90.19487 93.98) (end 86.925 97.24987) (width 0.2) (layer "F.Cu") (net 13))
 (segment (start 115.5 122.625) (end 117.63375 120.49125) (width 0.2) (layer "F.Cu") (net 13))
 (segment (start 86.925 97.24987) (end 86.925 122.625) (width 0.2) (layer "F.Cu") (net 13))
 (segment (start 117.63375 120.49125) (end 117.63375 111.76) (width 0.2) (layer "F.Cu") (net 13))
 (segment (start 86.925 122.625) (end 115.5 122.625) (width 0.2) (layer "F.Cu") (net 13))
 (segment (start 117.63375 92.71) (end 116.84 92.71) (width 0.2) (layer "F.Cu") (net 8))
 (segment (start 116.84 92.71) (end 107.95 101.6) (width 0.2) (layer "F.Cu") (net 8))
 (segment (start 107.95 101.6) (end 106.5125 101.6) (width 0.2) (layer "F.Cu") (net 8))
 (segment (start 130.96875 86.995) (end 130.96875 86.525) (width 0.2) (layer "F.Cu") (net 11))
 (segment (start 114.7 91.95013) (end 107.59013 99.06) (width 0.2) (layer "F.Cu") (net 11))
 (segment (start 107.59013 99.06) (end 106.5125 99.06) (width 0.2) (layer "F.Cu") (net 11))
 (segment (start 136.68375 92.71) (end 130.96875 86.995) (width 0.2) (layer "F.Cu") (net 11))
 (segment (start 114.7 86.525) (end 114.7 91.95013) (width 0.2) (layer "F.Cu") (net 11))
 (segment (start 130.96875 86.525) (end 114.7 86.525) (width 0.2) (layer "F.Cu") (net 11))
 (segment (start 150.01875 86.125) (end 114.3 86.125) (width 0.2) (layer "F.Cu") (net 9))
 (segment (start 114.3 89.5175) (end 107.2975 96.52) (width 0.2) (layer "F.Cu") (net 9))
 (segment (start 150.01875 87.3125) (end 150.01875 86.125) (width 0.2) (layer "F.Cu") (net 9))
 (segment (start 114.3 86.125) (end 114.3 89.5175) (width 0.2) (layer "F.Cu") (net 9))
 (segment (start 155.41625 92.71) (end 150.01875 87.3125) (width 0.2) (layer "F.Cu") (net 9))
 (segment (start 107.59013 93.98) (end 106.5125 93.98) (width 0.2) (layer "F.Cu") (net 6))
 (segment (start 174.46625 91.1225) (end 169.06875 85.725) (width 0.2) (layer "F.Cu") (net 6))
 (segment (start 169.06875 85.725) (end 111.91875 85.725) (width 0.2) (layer "F.Cu") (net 6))
 (segment (start 111.91875 89.65138) (end 107.59013 93.98) (width 0.2) (layer "F.Cu") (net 6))
 (segment (start 174.46625 92.71) (end 174.46625 91.1225) (width 0.2) (layer "F.Cu") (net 6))
 (segment (start 111.91875 85.725) (end 111.91875 89.65138) (width 0.2) (layer "F.Cu") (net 6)))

